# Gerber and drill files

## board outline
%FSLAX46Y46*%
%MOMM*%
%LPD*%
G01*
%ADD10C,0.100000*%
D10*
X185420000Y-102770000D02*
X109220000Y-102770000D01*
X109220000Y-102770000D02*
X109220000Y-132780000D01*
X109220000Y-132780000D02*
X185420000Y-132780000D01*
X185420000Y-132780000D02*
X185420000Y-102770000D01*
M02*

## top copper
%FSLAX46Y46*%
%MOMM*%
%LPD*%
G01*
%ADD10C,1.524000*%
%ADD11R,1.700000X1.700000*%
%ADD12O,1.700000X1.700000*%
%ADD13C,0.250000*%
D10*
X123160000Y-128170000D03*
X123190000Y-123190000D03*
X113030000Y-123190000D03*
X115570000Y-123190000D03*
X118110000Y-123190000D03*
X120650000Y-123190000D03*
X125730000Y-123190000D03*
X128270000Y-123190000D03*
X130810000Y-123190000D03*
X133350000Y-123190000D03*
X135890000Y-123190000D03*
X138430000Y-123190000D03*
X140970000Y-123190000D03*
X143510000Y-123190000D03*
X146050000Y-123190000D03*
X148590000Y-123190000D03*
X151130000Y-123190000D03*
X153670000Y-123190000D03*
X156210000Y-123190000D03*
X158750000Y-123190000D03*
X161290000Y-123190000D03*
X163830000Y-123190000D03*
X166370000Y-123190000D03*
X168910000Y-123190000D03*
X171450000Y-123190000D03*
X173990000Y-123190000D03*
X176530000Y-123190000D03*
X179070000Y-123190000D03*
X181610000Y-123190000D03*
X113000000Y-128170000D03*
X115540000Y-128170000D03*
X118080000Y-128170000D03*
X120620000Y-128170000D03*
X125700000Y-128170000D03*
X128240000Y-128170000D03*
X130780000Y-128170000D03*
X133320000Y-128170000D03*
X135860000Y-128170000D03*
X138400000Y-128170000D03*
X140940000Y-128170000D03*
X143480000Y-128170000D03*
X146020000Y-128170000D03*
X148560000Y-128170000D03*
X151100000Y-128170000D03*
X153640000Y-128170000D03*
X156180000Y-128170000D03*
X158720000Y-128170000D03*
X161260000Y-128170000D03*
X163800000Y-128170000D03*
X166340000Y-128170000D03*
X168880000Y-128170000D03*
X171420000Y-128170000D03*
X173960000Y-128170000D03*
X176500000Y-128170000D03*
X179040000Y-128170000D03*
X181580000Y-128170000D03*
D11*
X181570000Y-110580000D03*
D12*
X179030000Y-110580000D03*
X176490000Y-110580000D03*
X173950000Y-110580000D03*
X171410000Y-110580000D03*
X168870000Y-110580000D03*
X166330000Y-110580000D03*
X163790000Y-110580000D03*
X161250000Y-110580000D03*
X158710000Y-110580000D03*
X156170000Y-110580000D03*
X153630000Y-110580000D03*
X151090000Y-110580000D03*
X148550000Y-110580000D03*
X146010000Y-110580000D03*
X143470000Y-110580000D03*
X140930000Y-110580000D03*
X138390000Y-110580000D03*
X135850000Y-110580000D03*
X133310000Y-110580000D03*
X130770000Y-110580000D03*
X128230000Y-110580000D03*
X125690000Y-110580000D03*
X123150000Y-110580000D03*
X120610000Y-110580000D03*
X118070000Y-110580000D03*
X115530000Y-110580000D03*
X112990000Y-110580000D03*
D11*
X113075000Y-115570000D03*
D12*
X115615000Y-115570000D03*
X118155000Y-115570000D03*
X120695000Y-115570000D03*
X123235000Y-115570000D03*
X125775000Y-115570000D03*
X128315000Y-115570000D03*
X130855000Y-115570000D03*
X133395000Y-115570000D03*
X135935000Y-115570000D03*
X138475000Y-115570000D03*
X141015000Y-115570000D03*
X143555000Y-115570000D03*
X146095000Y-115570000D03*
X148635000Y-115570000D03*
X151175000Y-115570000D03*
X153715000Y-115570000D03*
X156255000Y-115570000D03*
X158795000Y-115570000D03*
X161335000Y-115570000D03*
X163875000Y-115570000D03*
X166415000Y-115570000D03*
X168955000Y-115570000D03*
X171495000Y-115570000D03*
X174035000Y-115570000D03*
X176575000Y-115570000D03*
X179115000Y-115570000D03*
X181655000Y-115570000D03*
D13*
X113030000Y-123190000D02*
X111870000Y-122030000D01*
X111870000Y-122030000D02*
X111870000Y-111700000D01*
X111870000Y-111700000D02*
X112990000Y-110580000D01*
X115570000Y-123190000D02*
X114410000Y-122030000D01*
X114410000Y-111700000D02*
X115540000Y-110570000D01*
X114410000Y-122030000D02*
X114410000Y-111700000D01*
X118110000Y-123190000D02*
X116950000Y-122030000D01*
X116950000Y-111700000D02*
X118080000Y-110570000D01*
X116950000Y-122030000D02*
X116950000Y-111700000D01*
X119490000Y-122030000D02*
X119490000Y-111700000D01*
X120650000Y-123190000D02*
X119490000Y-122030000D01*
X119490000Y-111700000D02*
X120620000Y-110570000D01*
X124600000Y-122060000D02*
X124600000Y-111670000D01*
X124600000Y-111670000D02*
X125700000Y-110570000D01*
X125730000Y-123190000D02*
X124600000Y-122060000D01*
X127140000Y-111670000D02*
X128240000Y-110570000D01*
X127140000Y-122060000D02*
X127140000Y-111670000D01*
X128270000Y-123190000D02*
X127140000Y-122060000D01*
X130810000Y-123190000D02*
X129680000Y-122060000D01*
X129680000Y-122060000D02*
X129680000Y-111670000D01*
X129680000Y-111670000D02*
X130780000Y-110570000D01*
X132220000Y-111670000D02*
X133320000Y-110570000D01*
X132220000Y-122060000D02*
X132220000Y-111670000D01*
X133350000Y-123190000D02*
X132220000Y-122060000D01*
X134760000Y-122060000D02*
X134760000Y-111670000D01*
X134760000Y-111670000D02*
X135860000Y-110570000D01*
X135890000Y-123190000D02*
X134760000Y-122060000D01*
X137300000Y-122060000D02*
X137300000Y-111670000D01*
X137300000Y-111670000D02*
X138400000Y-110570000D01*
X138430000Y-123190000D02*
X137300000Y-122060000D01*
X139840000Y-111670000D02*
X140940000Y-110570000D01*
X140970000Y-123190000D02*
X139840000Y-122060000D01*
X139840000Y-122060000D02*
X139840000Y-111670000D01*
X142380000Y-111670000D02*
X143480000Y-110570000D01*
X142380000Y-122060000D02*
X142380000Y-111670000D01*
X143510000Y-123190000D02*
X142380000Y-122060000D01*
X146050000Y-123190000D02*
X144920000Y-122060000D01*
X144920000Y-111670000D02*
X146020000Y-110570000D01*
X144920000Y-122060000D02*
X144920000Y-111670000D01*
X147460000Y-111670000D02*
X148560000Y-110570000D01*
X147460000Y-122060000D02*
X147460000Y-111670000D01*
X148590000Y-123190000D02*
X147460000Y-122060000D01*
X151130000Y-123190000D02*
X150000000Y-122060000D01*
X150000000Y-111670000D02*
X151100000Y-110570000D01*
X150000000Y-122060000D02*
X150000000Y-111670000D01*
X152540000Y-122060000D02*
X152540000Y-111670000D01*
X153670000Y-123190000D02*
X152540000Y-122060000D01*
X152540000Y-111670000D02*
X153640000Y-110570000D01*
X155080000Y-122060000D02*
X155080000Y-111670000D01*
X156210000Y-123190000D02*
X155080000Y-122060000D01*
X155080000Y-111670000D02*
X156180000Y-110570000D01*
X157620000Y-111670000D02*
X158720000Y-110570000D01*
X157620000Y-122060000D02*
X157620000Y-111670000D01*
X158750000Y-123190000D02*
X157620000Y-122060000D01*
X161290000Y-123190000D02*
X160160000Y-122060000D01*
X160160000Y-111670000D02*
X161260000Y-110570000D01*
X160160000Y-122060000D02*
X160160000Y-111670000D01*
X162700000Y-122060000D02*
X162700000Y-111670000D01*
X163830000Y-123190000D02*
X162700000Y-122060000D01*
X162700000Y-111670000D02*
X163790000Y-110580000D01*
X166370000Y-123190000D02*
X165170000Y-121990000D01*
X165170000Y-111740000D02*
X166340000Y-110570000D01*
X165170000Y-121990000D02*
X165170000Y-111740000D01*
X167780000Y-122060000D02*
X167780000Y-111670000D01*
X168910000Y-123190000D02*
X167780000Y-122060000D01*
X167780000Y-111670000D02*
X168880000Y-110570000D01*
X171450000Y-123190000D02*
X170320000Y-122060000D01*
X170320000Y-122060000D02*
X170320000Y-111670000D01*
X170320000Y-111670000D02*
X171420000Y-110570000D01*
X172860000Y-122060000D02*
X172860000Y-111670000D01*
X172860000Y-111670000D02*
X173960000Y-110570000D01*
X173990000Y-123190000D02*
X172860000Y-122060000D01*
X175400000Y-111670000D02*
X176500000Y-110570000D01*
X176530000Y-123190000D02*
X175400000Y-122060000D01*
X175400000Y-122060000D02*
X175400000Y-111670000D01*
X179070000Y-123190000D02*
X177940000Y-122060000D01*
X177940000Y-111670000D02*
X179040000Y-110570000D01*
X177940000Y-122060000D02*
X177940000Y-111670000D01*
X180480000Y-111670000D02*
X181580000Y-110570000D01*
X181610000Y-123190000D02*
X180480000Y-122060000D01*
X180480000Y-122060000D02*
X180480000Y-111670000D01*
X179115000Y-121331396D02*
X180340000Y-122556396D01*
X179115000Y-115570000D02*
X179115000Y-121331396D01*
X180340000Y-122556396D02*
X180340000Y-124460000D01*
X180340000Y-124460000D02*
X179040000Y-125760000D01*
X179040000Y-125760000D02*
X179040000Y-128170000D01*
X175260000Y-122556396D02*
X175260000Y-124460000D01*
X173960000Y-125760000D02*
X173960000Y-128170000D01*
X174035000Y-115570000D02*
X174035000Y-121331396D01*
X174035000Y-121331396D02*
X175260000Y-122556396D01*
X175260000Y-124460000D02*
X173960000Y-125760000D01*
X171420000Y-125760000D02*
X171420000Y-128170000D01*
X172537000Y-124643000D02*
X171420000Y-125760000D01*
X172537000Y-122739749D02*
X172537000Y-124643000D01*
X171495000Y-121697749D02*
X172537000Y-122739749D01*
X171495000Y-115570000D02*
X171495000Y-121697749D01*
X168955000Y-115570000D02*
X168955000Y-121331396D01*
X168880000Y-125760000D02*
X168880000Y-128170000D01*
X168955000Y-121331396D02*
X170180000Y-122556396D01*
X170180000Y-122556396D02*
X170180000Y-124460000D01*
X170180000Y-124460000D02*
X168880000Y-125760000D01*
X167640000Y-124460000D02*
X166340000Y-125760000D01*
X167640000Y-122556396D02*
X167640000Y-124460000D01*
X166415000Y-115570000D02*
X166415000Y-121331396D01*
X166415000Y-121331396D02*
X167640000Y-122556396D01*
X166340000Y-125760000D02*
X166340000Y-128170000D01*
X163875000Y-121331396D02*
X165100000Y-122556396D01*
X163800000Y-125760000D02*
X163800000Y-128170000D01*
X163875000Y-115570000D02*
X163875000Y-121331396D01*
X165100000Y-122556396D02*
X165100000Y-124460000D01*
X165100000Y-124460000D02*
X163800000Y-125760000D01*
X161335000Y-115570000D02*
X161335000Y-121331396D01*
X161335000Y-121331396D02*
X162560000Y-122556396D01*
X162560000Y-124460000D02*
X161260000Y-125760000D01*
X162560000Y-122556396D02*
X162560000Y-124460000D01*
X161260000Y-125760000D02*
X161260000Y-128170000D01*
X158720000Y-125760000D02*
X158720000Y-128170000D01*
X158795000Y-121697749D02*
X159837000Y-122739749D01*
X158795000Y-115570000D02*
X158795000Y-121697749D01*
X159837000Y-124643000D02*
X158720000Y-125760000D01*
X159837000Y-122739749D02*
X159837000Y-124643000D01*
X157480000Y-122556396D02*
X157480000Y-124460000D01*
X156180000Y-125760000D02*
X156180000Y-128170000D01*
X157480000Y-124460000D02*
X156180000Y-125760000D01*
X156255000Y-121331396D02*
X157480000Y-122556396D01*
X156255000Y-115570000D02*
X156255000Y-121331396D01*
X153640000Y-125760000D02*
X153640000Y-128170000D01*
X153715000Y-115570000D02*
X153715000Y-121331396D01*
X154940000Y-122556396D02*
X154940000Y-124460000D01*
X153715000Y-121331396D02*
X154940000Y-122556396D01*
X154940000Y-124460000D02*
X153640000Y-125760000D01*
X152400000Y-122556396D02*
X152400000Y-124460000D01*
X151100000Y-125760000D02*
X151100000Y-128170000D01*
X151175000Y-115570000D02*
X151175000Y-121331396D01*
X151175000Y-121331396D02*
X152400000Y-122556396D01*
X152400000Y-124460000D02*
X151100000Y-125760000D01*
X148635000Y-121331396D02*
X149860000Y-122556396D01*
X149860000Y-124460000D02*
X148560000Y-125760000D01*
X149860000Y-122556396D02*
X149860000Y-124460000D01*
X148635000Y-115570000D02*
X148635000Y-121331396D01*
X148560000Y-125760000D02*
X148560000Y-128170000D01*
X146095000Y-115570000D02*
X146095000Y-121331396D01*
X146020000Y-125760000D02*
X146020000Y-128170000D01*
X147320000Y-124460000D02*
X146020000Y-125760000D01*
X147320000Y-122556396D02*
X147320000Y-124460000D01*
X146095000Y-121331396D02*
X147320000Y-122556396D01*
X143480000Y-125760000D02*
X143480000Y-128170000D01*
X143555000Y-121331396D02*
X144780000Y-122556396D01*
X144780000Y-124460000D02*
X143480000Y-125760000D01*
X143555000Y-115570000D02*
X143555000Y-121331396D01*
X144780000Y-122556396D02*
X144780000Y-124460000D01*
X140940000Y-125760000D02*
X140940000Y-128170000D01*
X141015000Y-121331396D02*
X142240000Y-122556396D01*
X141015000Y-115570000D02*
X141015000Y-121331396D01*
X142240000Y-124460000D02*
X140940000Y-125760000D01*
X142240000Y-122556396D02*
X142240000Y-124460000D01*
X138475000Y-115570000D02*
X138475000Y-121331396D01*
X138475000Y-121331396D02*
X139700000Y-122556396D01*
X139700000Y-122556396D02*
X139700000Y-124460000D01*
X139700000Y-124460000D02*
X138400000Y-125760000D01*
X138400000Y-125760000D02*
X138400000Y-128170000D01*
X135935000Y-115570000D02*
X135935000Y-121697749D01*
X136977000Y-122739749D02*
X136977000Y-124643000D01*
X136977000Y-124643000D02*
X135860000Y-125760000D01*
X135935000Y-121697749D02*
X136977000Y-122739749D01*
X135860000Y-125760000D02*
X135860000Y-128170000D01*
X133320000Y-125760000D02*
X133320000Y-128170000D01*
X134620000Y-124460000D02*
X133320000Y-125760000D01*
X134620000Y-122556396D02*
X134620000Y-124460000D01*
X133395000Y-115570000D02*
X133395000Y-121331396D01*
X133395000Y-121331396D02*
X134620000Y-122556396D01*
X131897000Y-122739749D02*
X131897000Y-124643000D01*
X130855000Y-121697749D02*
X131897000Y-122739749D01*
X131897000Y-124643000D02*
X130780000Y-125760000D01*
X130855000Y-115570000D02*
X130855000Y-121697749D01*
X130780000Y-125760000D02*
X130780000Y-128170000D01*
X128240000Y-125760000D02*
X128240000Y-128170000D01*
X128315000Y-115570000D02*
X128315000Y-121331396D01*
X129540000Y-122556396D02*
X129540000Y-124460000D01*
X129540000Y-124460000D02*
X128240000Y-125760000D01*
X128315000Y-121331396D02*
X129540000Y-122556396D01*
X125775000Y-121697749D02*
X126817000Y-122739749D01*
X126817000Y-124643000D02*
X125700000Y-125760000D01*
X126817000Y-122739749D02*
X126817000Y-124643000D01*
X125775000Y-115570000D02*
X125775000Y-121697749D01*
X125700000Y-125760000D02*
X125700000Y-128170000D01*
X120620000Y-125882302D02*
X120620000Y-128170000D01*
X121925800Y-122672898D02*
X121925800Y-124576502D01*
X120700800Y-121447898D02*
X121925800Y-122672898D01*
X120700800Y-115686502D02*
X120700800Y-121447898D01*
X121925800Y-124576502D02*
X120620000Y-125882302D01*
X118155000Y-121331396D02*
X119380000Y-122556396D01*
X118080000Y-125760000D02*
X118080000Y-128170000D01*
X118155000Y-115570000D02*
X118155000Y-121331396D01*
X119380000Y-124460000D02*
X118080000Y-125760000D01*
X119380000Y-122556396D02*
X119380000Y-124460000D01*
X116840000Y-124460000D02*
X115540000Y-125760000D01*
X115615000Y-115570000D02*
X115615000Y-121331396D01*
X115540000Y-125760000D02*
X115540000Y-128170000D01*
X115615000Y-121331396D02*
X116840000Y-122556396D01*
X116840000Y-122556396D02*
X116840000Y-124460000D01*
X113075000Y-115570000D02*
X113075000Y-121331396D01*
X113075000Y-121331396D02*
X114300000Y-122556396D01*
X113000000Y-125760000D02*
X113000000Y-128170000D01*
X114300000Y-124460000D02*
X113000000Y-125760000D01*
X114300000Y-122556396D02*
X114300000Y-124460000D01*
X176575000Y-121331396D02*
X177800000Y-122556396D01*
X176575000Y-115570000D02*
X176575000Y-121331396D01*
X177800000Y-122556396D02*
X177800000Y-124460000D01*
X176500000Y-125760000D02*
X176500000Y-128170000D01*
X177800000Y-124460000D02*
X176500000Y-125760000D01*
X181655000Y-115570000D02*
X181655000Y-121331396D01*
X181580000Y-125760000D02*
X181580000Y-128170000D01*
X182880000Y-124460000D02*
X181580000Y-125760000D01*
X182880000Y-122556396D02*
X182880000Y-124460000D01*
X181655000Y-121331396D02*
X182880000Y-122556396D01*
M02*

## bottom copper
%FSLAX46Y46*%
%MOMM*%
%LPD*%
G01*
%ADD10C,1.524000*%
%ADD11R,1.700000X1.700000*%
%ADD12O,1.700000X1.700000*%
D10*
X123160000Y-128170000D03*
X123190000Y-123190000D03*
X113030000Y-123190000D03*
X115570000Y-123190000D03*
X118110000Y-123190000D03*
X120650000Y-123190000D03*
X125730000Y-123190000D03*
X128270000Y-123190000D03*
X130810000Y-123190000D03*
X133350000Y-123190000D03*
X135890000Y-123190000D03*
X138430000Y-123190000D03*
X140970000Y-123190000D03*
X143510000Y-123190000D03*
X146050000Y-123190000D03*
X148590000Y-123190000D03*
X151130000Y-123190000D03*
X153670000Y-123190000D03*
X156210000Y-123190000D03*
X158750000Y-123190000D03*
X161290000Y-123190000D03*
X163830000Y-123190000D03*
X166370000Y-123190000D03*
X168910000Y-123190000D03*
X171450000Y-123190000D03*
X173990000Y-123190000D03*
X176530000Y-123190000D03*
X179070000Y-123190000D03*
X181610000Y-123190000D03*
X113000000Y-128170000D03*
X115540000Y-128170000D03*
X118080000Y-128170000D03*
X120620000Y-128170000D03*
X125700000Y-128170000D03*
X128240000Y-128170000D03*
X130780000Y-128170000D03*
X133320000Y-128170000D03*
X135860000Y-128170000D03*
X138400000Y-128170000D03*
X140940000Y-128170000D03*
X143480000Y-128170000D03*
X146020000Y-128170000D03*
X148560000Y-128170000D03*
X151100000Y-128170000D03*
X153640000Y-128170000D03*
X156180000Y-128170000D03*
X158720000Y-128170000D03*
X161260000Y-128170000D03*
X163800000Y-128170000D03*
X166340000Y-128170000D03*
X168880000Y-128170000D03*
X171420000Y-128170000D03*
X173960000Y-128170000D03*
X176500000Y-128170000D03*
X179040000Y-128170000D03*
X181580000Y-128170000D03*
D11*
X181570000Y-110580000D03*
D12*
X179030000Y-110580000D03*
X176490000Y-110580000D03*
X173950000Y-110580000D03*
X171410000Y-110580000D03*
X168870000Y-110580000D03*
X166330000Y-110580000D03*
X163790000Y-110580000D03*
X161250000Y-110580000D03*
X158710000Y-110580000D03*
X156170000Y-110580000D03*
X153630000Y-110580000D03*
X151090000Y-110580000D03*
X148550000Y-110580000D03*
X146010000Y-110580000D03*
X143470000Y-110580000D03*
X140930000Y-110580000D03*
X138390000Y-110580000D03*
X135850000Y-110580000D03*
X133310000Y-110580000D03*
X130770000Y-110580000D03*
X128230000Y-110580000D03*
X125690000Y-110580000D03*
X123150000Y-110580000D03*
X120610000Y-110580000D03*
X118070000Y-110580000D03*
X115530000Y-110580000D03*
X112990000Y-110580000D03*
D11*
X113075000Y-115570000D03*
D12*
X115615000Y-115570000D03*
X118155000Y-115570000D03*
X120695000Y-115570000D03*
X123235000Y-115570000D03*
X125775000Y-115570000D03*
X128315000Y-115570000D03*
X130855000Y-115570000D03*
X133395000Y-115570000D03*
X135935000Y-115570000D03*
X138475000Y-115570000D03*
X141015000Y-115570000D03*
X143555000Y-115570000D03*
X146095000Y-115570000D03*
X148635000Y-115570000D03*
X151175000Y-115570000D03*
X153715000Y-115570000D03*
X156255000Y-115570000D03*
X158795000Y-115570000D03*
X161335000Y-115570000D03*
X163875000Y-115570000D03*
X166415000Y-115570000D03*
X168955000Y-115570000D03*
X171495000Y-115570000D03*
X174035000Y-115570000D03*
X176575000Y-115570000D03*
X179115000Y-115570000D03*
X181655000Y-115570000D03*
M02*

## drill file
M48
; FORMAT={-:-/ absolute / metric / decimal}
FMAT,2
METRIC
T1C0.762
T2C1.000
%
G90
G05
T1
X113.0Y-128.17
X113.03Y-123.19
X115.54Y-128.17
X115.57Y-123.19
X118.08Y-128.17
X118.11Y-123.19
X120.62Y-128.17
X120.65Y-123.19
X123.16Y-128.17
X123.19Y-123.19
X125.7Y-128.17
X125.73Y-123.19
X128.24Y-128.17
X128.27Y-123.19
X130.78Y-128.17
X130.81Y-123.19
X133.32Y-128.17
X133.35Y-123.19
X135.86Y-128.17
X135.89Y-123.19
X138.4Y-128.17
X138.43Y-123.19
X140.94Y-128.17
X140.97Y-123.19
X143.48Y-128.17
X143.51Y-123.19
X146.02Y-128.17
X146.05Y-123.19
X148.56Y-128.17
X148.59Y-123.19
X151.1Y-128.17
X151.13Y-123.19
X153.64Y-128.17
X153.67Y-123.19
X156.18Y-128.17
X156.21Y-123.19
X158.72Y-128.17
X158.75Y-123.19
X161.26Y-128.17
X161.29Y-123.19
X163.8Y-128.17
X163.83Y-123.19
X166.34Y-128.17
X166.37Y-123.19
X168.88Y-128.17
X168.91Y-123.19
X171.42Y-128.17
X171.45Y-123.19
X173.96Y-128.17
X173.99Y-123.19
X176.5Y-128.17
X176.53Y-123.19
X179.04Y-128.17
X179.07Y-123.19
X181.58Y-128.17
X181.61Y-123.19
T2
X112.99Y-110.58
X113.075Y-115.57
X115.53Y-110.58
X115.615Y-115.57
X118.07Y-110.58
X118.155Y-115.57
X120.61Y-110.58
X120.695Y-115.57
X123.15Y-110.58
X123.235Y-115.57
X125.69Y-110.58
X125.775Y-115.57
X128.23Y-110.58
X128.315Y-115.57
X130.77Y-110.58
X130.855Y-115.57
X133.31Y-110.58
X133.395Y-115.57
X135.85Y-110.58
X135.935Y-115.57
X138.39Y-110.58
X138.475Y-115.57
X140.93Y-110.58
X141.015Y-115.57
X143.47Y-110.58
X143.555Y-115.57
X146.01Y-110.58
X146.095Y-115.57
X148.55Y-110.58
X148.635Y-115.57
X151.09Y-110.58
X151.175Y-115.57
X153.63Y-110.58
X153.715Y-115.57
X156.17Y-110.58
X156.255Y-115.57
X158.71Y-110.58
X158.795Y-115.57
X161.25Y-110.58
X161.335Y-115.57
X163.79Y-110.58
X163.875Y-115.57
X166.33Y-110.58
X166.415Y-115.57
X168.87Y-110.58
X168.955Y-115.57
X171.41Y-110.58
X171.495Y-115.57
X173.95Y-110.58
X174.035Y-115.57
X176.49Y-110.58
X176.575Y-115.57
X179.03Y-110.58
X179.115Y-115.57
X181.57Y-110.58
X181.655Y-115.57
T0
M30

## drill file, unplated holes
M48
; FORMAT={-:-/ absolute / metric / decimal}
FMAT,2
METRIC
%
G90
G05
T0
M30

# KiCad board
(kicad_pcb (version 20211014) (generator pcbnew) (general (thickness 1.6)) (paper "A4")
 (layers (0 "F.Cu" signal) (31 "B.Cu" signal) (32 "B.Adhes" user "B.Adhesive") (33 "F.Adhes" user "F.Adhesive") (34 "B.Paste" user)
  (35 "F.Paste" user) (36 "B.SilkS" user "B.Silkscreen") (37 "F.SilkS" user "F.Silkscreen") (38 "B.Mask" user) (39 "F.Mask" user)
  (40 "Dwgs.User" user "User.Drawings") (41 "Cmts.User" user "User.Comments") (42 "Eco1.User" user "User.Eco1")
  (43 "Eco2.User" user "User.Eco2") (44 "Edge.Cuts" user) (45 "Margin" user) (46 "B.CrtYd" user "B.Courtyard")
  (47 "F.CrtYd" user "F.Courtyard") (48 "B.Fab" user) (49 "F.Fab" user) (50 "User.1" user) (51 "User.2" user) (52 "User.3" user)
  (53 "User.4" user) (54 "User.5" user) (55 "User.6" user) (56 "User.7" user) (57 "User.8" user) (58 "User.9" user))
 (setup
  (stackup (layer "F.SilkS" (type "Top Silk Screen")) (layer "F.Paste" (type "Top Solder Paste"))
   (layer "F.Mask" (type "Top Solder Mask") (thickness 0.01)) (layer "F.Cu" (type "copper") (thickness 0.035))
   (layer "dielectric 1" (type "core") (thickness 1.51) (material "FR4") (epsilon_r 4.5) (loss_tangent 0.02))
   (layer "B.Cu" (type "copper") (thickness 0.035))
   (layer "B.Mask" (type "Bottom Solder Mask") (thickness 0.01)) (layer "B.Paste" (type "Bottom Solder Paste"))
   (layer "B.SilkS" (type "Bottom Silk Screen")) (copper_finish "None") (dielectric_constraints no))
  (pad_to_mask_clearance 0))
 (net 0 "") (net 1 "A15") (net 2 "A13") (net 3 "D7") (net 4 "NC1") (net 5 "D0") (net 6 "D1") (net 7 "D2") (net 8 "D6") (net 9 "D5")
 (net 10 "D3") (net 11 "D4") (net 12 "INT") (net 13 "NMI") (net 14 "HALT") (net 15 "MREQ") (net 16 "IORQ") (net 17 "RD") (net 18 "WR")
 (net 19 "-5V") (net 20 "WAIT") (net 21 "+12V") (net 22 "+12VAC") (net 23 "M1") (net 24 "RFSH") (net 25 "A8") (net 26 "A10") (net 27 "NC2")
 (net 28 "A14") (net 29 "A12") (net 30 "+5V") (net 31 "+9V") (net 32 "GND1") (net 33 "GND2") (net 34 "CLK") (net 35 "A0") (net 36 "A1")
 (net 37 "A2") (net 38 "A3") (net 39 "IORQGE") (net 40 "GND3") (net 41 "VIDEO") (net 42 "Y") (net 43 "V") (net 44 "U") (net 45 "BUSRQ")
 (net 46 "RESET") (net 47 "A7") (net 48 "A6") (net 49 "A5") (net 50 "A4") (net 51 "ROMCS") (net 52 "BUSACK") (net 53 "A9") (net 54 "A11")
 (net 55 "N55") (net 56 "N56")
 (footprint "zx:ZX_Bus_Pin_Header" (layer "F.Cu") (at 147.32 124.46)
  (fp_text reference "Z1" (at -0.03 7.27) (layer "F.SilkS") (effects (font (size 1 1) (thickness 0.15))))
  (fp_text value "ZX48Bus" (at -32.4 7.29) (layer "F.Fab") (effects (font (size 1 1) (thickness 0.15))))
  (pad "" thru_hole circle (at -24.16 3.71) (size 1.524 1.524) (drill 0.762) (layers *.Cu *.Mask))
  (pad "" thru_hole circle (at -24.13 -1.27) (size 1.524 1.524) (drill 0.762) (layers *.Cu *.Mask))
  (pad "A1" thru_hole circle (at -34.29 -1.27) (size 1.524 1.524) (drill 0.762) (layers *.Cu *.Mask) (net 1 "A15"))
  (pad "A2" thru_hole circle (at -31.75 -1.27) (size 1.524 1.524) (drill 0.762) (layers *.Cu *.Mask) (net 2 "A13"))
  (pad "A3" thru_hole circle (at -29.21 -1.27) (size 1.524 1.524) (drill 0.762) (layers *.Cu *.Mask) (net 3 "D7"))
  (pad "A4" thru_hole circle (at -26.67 -1.27) (size 1.524 1.524) (drill 0.762) (layers *.Cu *.Mask) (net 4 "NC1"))
  (pad "A6" thru_hole circle (at -21.59 -1.27) (size 1.524 1.524) (drill 0.762) (layers *.Cu *.Mask) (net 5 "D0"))
  (pad "A7" thru_hole circle (at -19.05 -1.27) (size 1.524 1.524) (drill 0.762) (layers *.Cu *.Mask) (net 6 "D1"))
  (pad "A8" thru_hole circle (at -16.51 -1.27) (size 1.524 1.524) (drill 0.762) (layers *.Cu *.Mask) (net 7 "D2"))
  (pad "A9" thru_hole circle (at -13.97 -1.27) (size 1.524 1.524) (drill 0.762) (layers *.Cu *.Mask) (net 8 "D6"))
  (pad "A10" thru_hole circle (at -11.43 -1.27) (size 1.524 1.524) (drill 0.762) (layers *.Cu *.Mask) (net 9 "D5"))
  (pad "A11" thru_hole circle (at -8.89 -1.27) (size 1.524 1.524) (drill 0.762) (layers *.Cu *.Mask) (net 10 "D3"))
  (pad "A12" thru_hole circle (at -6.35 -1.27) (size 1.524 1.524) (drill 0.762) (layers *.Cu *.Mask) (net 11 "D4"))
  (pad "A13" thru_hole circle (at -3.81 -1.27) (size 1.524 1.524) (drill 0.762) (layers *.Cu *.Mask) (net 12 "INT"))
  (pad "A14" thru_hole circle (at -1.27 -1.27) (size 1.524 1.524) (drill 0.762) (layers *.Cu *.Mask) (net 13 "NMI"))
  (pad "A15" thru_hole circle (at 1.27 -1.27) (size 1.524 1.524) (drill 0.762) (layers *.Cu *.Mask) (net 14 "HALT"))
  (pad "A16" thru_hole circle (at 3.81 -1.27) (size 1.524 1.524) (drill 0.762) (layers *.Cu *.Mask) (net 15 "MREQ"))
  (pad "A17" thru_hole circle (at 6.35 -1.27) (size 1.524 1.524) (drill 0.762) (layers *.Cu *.Mask) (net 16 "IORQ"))
  (pad "A18" thru_hole circle (at 8.89 -1.27) (size 1.524 1.524) (drill 0.762) (layers *.Cu *.Mask) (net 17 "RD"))
  (pad "A19" thru_hole circle (at 11.43 -1.27) (size 1.524 1.524) (drill 0.762) (layers *.Cu *.Mask) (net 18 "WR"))
  (pad "A20" thru_hole circle (at 13.97 -1.27) (size 1.524 1.524) (drill 0.762) (layers *.Cu *.Mask) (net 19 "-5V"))
  (pad "A21" thru_hole circle (at 16.51 -1.27) (size 1.524 1.524) (drill 0.762) (layers *.Cu *.Mask) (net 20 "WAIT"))
  (pad "A22" thru_hole circle (at 19.05 -1.27) (size 1.524 1.524) (drill 0.762) (layers *.Cu *.Mask) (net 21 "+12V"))
  (pad "A23" thru_hole circle (at 21.59 -1.27) (size 1.524 1.524) (drill 0.762) (layers *.Cu *.Mask) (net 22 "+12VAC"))
  (pad "A24" thru_hole circle (at 24.13 -1.27) (size 1.524 1.524) (drill 0.762) (layers *.Cu *.Mask) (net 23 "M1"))
  (pad "A25" thru_hole circle (at 26.67 -1.27) (size 1.524 1.524) (drill 0.762) (layers *.Cu *.Mask) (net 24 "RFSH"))
  (pad "A26" thru_hole circle (at 29.21 -1.27) (size 1.524 1.524) (drill 0.762) (layers *.Cu *.Mask) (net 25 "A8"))
  (pad "A27" thru_hole circle (at 31.75 -1.27) (size 1.524 1.524) (drill 0.762) (layers *.Cu *.Mask) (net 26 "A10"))
  (pad "A28" thru_hole circle (at 34.29 -1.27) (size 1.524 1.524) (drill 0.762) (layers *.Cu *.Mask) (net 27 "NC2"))
  (pad "B1" thru_hole circle (at -34.32 3.71) (size 1.524 1.524) (drill 0.762) (layers *.Cu *.Mask) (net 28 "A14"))
  (pad "B2" thru_hole circle (at -31.78 3.71) (size 1.524 1.524) (drill 0.762) (layers *.Cu *.Mask) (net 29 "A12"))
  (pad "B3" thru_hole circle (at -29.24 3.71) (size 1.524 1.524) (drill 0.762) (layers *.Cu *.Mask) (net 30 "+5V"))
  (pad "B4" thru_hole circle (at -26.7 3.71) (size 1.524 1.524) (drill 0.762) (layers *.Cu *.Mask) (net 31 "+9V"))
  (pad "B6" thru_hole circle (at -21.62 3.71) (size 1.524 1.524) (drill 0.762) (layers *.Cu *.Mask) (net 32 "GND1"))
  (pad "B7" thru_hole circle (at -19.08 3.71) (size 1.524 1.524) (drill 0.762) (layers *.Cu *.Mask) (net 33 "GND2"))
  (pad "B8" thru_hole circle (at -16.54 3.71) (size 1.524 1.524) (drill 0.762) (layers *.Cu *.Mask) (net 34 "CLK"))
  (pad "B9" thru_hole circle (at -14 3.71) (size 1.524 1.524) (drill 0.762) (layers *.Cu *.Mask) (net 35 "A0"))
  (pad "B10" thru_hole circle (at -11.46 3.71) (size 1.524 1.524) (drill 0.762) (layers *.Cu *.Mask) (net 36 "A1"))
  (pad "B11" thru_hole circle (at -8.92 3.71) (size 1.524 1.524) (drill 0.762) (layers *.Cu *.Mask) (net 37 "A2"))
  (pad "B12" thru_hole circle (at -6.38 3.71) (size 1.524 1.524) (drill 0.762) (layers *.Cu *.Mask) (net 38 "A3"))
  (pad "B13" thru_hole circle (at -3.84 3.71) (size 1.524 1.524) (drill 0.762) (layers *.Cu *.Mask) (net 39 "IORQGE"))
  (pad "B14" thru_hole circle (at -1.3 3.71) (size 1.524 1.524) (drill 0.762) (layers *.Cu *.Mask) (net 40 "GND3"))
  (pad "B15" thru_hole circle (at 1.24 3.71) (size 1.524 1.524) (drill 0.762) (layers *.Cu *.Mask) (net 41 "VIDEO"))
  (pad "B16" thru_hole circle (at 3.78 3.71) (size 1.524 1.524) (drill 0.762) (layers *.Cu *.Mask) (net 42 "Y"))
  (pad "B17" thru_hole circle (at 6.32 3.71) (size 1.524 1.524) (drill 0.762) (layers *.Cu *.Mask) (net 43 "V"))
  (pad "B18" thru_hole circle (at 8.86 3.71) (size 1.524 1.524) (drill 0.762) (layers *.Cu *.Mask) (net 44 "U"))
  (pad "B19" thru_hole circle (at 11.4 3.71) (size 1.524 1.524) (drill 0.762) (layers *.Cu *.Mask) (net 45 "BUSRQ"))
  (pad "B20" thru_hole circle (at 13.94 3.71) (size 1.524 1.524) (drill 0.762) (layers *.Cu *.Mask) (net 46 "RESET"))
  (pad "B21" thru_hole circle (at 16.48 3.71) (size 1.524 1.524) (drill 0.762) (layers *.Cu *.Mask) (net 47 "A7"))
  (pad "B22" thru_hole circle (at 19.02 3.71) (size 1.524 1.524) (drill 0.762) (layers *.Cu *.Mask) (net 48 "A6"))
  (pad "B23" thru_hole circle (at 21.56 3.71) (size 1.524 1.524) (drill 0.762) (layers *.Cu *.Mask) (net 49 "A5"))
  (pad "B24" thru_hole circle (at 24.1 3.71) (size 1.524 1.524) (drill 0.762) (layers *.Cu *.Mask) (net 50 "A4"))
  (pad "B25" thru_hole circle (at 26.64 3.71) (size 1.524 1.524) (drill 0.762) (layers *.Cu *.Mask) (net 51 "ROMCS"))
  (pad "B26" thru_hole circle (at 29.18 3.71) (size 1.524 1.524) (drill 0.762) (layers *.Cu *.Mask) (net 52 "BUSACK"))
  (pad "B27" thru_hole circle (at 31.72 3.71) (size 1.524 1.524) (drill 0.762) (layers *.Cu *.Mask) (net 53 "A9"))
  (pad "B28" thru_hole circle (at 34.26 3.71) (size 1.524 1.524) (drill 0.762) (layers *.Cu *.Mask) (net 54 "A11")))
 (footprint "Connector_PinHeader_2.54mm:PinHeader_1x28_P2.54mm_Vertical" (layer "B.Cu") (at 181.57 110.58 90)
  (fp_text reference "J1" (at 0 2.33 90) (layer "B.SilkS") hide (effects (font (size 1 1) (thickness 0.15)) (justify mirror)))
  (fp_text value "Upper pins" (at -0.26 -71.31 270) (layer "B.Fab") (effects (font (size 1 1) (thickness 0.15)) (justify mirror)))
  (pad "1" thru_hole rect (at 0 0 90) (size 1.7 1.7) (drill 1) (layers *.Cu *.Mask) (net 27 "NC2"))
  (pad "2" thru_hole oval (at 0 -2.54 90) (size 1.7 1.7) (drill 1) (layers *.Cu *.Mask) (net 26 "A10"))
  (pad "3" thru_hole oval (at 0 -5.08 90) (size 1.7 1.7) (drill 1) (layers *.Cu *.Mask) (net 25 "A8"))
  (pad "4" thru_hole oval (at 0 -7.62 90) (size 1.7 1.7) (drill 1) (layers *.Cu *.Mask) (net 24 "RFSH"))
  (pad "5" thru_hole oval (at 0 -10.16 90) (size 1.7 1.7) (drill 1) (layers *.Cu *.Mask) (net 23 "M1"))
  (pad "6" thru_hole oval (at 0 -12.7 90) (size 1.7 1.7) (drill 1) (layers *.Cu *.Mask) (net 22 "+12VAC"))
  (pad "7" thru_hole oval (at 0 -15.24 90) (size 1.7 1.7) (drill 1) (layers *.Cu *.Mask) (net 21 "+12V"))
  (pad "8" thru_hole oval (at 0 -17.78 90) (size 1.7 1.7) (drill 1) (layers *.Cu *.Mask) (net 20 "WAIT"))
  (pad "9" thru_hole oval (at 0 -20.32 90) (size 1.7 1.7) (drill 1) (layers *.Cu *.Mask) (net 19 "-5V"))
  (pad "10" thru_hole oval (at 0 -22.86 90) (size 1.7 1.7) (drill 1) (layers *.Cu *.Mask) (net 18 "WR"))
  (pad "11" thru_hole oval (at 0 -25.4 90) (size 1.7 1.7) (drill 1) (layers *.Cu *.Mask) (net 17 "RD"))
  (pad "12" thru_hole oval (at 0 -27.94 90) (size 1.7 1.7) (drill 1) (layers *.Cu *.Mask) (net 16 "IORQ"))
  (pad "13" thru_hole oval (at 0 -30.48 90) (size 1.7 1.7) (drill 1) (layers *.Cu *.Mask) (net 15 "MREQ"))
  (pad "14" thru_hole oval (at 0 -33.02 90) (size 1.7 1.7) (drill 1) (layers *.Cu *.Mask) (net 14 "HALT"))
  (pad "15" thru_hole oval (at 0 -35.56 90) (size 1.7 1.7) (drill 1) (layers *.Cu *.Mask) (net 13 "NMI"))
  (pad "16" thru_hole oval (at 0 -38.1 90) (size 1.7 1.7) (drill 1) (layers *.Cu *.Mask) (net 12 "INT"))
  (pad "17" thru_hole oval (at 0 -40.64 90) (size 1.7 1.7) (drill 1) (layers *.Cu *.Mask) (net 11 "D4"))
  (pad "18" thru_hole oval (at 0 -43.18 90) (size 1.7 1.7) (drill 1) (layers *.Cu *.Mask) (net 10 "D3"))
  (pad "19" thru_hole oval (at 0 -45.72 90) (size 1.7 1.7) (drill 1) (layers *.Cu *.Mask) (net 9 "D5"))
  (pad "20" thru_hole oval (at 0 -48.26 90) (size 1.7 1.7) (drill 1) (layers *.Cu *.Mask) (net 8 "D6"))
  (pad "21" thru_hole oval (at 0 -50.8 90) (size 1.7 1.7) (drill 1) (layers *.Cu *.Mask) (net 7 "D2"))
  (pad "22" thru_hole oval (at 0 -53.34 90) (size 1.7 1.7) (drill 1) (layers *.Cu *.Mask) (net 6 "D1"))
  (pad "23" thru_hole oval (at 0 -55.88 90) (size 1.7 1.7) (drill 1) (layers *.Cu *.Mask) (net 5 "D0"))
  (pad "24" thru_hole oval (at 0 -58.42 90) (size 1.7 1.7) (drill 1) (layers *.Cu *.Mask) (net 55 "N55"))
  (pad "25" thru_hole oval (at 0 -60.96 90) (size 1.7 1.7) (drill 1) (layers *.Cu *.Mask) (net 4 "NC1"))
  (pad "26" thru_hole oval (at 0 -63.5 90) (size 1.7 1.7) (drill 1) (layers *.Cu *.Mask) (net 3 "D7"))
  (pad "27" thru_hole oval (at 0 -66.04 90) (size 1.7 1.7) (drill 1) (layers *.Cu *.Mask) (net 2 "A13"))
  (pad "28" thru_hole oval (at 0 -68.58 90) (size 1.7 1.7) (drill 1) (layers *.Cu *.Mask) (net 1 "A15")))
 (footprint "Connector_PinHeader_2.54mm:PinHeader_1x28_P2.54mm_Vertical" (layer "B.Cu") (at 113.075 115.57 -90)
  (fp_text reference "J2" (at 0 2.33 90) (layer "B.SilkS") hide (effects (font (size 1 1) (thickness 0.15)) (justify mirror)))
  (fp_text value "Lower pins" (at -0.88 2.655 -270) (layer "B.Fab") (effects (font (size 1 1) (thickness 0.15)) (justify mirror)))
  (pad "1" thru_hole rect (at 0 0 270) (size 1.7 1.7) (drill 1) (layers *.Cu *.Mask) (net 28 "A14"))
  (pad "2" thru_hole oval (at 0 -2.54 270) (size 1.7 1.7) (drill 1) (layers *.Cu *.Mask) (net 29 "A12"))
  (pad "3" thru_hole oval (at 0 -5.08 270) (size 1.7 1.7) (drill 1) (layers *.Cu *.Mask) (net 30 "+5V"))
  (pad "4" thru_hole oval (at 0 -7.62 270) (size 1.7 1.7) (drill 1) (layers *.Cu *.Mask) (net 31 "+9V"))
  (pad "5" thru_hole oval (at 0 -10.16 270) (size 1.7 1.7) (drill 1) (layers *.Cu *.Mask) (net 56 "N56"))
  (pad "6" thru_hole oval (at 0 -12.7 270) (size 1.7 1.7) (drill 1) (layers *.Cu *.Mask) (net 32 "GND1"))
  (pad "7" thru_hole oval (at 0 -15.24 270) (size 1.7 1.7) (drill 1) (layers *.Cu *.Mask) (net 33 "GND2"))
  (pad "8" thru_hole oval (at 0 -17.78 270) (size 1.7 1.7) (drill 1) (layers *.Cu *.Mask) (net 34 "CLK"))
  (pad "9" thru_hole oval (at 0 -20.32 270) (size 1.7 1.7) (drill 1) (layers *.Cu *.Mask) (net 35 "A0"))
  (pad "10" thru_hole oval (at 0 -22.86 270) (size 1.7 1.7) (drill 1) (layers *.Cu *.Mask) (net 36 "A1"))
  (pad "11" thru_hole oval (at 0 -25.4 270) (size 1.7 1.7) (drill 1) (layers *.Cu *.Mask) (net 37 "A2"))
  (pad "12" thru_hole oval (at 0 -27.94 270) (size 1.7 1.7) (drill 1) (layers *.Cu *.Mask) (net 38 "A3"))
  (pad "13" thru_hole oval (at 0 -30.48 270) (size 1.7 1.7) (drill 1) (layers *.Cu *.Mask) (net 39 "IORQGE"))
  (pad "14" thru_hole oval (at 0 -33.02 270) (size 1.7 1.7) (drill 1) (layers *.Cu *.Mask) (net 40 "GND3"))
  (pad "15" thru_hole oval (at 0 -35.56 270) (size 1.7 1.7) (drill 1) (layers *.Cu *.Mask) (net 41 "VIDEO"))
  (pad "16" thru_hole oval (at 0 -38.1 270) (size 1.7 1.7) (drill 1) (layers *.Cu *.Mask) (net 42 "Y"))
  (pad "17" thru_hole oval (at 0 -40.64 270) (size 1.7 1.7) (drill 1) (layers *.Cu *.Mask) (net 43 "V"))
  (pad "18" thru_hole oval (at 0 -43.18 270) (size 1.7 1.7) (drill 1) (layers *.Cu *.Mask) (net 44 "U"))
  (pad "19" thru_hole oval (at 0 -45.72 270) (size 1.7 1.7) (drill 1) (layers *.Cu *.Mask) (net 45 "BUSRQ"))
  (pad "20" thru_hole oval (at 0 -48.26 270) (size 1.7 1.7) (drill 1) (layers *.Cu *.Mask) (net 46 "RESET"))
  (pad "21" thru_hole oval (at 0 -50.8 270) (size 1.7 1.7) (drill 1) (layers *.Cu *.Mask) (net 47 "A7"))
  (pad "22" thru_hole oval (at 0 -53.34 270) (size 1.7 1.7) (drill 1) (layers *.Cu *.Mask) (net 48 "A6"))
  (pad "23" thru_hole oval (at 0 -55.88 270) (size 1.7 1.7) (drill 1) (layers *.Cu *.Mask) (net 49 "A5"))
  (pad "24" thru_hole oval (at 0 -58.42 270) (size 1.7 1.7) (drill 1) (layers *.Cu *.Mask) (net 50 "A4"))
  (pad "25" thru_hole oval (at 0 -60.96 270) (size 1.7 1.7) (drill 1) (layers *.Cu *.Mask) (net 51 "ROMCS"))
  (pad "26" thru_hole oval (at 0 -63.5 270) (size 1.7 1.7) (drill 1) (layers *.Cu *.Mask) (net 52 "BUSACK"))
  (pad "27" thru_hole oval (at 0 -66.04 270) (size 1.7 1.7) (drill 1) (layers *.Cu *.Mask) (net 53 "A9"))
  (pad "28" thru_hole oval (at 0 -68.58 270) (size 1.7 1.7) (drill 1) (layers *.Cu *.Mask) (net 54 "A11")))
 (gr_rect (start 185.42 102.77) (end 109.22 132.78) (layer "Edge.Cuts") (width 0.1) (fill none))
 (segment (start 113.03 123.19) (end 111.87 122.03) (width 0.25) (layer "F.Cu") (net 1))
 (segment (start 111.87 122.03) (end 111.87 111.7) (width 0.25) (layer "F.Cu") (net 1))
 (segment (start 111.87 111.7) (end 112.99 110.58) (width 0.25) (layer "F.Cu") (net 1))
 (segment (start 115.57 123.19) (end 114.41 122.03) (width 0.25) (layer "F.Cu") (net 2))
 (segment (start 114.41 111.7) (end 115.54 110.57) (width 0.25) (layer "F.Cu") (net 2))
 (segment (start 114.41 122.03) (end 114.41 111.7) (width 0.25) (layer "F.Cu") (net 2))
 (segment (start 118.11 123.19) (end 116.95 122.03) (width 0.25) (layer "F.Cu") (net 3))
 (segment (start 116.95 111.7) (end 118.08 110.57) (width 0.25) (layer "F.Cu") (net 3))
 (segment (start 116.95 122.03) (end 116.95 111.7) (width 0.25) (layer "F.Cu") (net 3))
 (segment (start 119.49 122.03) (end 119.49 111.7) (width 0.25) (layer "F.Cu") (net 4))
 (segment (start 120.65 123.19) (end 119.49 122.03) (width 0.25) (layer "F.Cu") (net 4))
 (segment (start 119.49 111.7) (end 120.62 110.57) (width 0.25) (layer "F.Cu") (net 4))
 (segment (start 124.6 122.06) (end 124.6 111.67) (width 0.25) (layer "F.Cu") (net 5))
 (segment (start 124.6 111.67) (end 125.7 110.57) (width 0.25) (layer "F.Cu") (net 5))
 (segment (start 125.73 123.19) (end 124.6 122.06) (width 0.25) (layer "F.Cu") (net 5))
 (segment (start 127.14 111.67) (end 128.24 110.57) (width 0.25) (layer "F.Cu") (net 6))
 (segment (start 127.14 122.06) (end 127.14 111.67) (width 0.25) (layer "F.Cu") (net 6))
 (segment (start 128.27 123.19) (end 127.14 122.06) (width 0.25) (layer "F.Cu") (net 6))
 (segment (start 130.81 123.19) (end 129.68 122.06) (width 0.25) (layer "F.Cu") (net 7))
 (segment (start 129.68 122.06) (end 129.68 111.67) (width 0.25) (layer "F.Cu") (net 7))
 (segment (start 129.68 111.67) (end 130.78 110.57) (width 0.25) (layer "F.Cu") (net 7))
 (segment (start 132.22 111.67) (end 133.32 110.57) (width 0.25) (layer "F.Cu") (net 8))
 (segment (start 132.22 122.06) (end 132.22 111.67) (width 0.25) (layer "F.Cu") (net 8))
 (segment (start 133.35 123.19) (end 132.22 122.06) (width 0.25) (layer "F.Cu") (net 8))
 (segment (start 134.76 122.06) (end 134.76 111.67) (width 0.25) (layer "F.Cu") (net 9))
 (segment (start 134.76 111.67) (end 135.86 110.57) (width 0.25) (layer "F.Cu") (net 9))
 (segment (start 135.89 123.19) (end 134.76 122.06) (width 0.25) (layer "F.Cu") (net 9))
 (segment (start 137.3 122.06) (end 137.3 111.67) (width 0.25) (layer "F.Cu") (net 10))
 (segment (start 137.3 111.67) (end 138.4 110.57) (width 0.25) (layer "F.Cu") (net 10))
 (segment (start 138.43 123.19) (end 137.3 122.06) (width 0.25) (layer "F.Cu") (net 10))
 (segment (start 139.84 111.67) (end 140.94 110.57) (width 0.25) (layer "F.Cu") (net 11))
 (segment (start 140.97 123.19) (end 139.84 122.06) (width 0.25) (layer "F.Cu") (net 11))
 (segment (start 139.84 122.06) (end 139.84 111.67) (width 0.25) (layer "F.Cu") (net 11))
 (segment (start 142.38 111.67) (end 143.48 110.57) (width 0.25) (layer "F.Cu") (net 12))
 (segment (start 142.38 122.06) (end 142.38 111.67) (width 0.25) (layer "F.Cu") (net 12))
 (segment (start 143.51 123.19) (end 142.38 122.06) (width 0.25) (layer "F.Cu") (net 12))
 (segment (start 146.05 123.19) (end 144.92 122.06) (width 0.25) (layer "F.Cu") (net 13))
 (segment (start 144.92 111.67) (end 146.02 110.57) (width 0.25) (layer "F.Cu") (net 13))
 (segment (start 144.92 122.06) (end 144.92 111.67) (width 0.25) (layer "F.Cu") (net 13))
 (segment (start 147.46 111.67) (end 148.56 110.57) (width 0.25) (layer "F.Cu") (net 14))
 (segment (start 147.46 122.06) (end 147.46 111.67) (width 0.25) (layer "F.Cu") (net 14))
 (segment (start 148.59 123.19) (end 147.46 122.06) (width 0.25) (layer "F.Cu") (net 14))
 (segment (start 151.13 123.19) (end 150 122.06) (width 0.25) (layer "F.Cu") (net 15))
 (segment (start 150 111.67) (end 151.1 110.57) (width 0.25) (layer "F.Cu") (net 15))
 (segment (start 150 122.06) (end 150 111.67) (width 0.25) (layer "F.Cu") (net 15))
 (segment (start 152.54 122.06) (end 152.54 111.67) (width 0.25) (layer "F.Cu") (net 16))
 (segment (start 153.67 123.19) (end 152.54 122.06) (width 0.25) (layer "F.Cu") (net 16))
 (segment (start 152.54 111.67) (end 153.64 110.57) (width 0.25) (layer "F.Cu") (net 16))
 (segment (start 155.08 122.06) (end 155.08 111.67) (width 0.25) (layer "F.Cu") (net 17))
 (segment (start 156.21 123.19) (end 155.08 122.06) (width 0.25) (layer "F.Cu") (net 17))
 (segment (start 155.08 111.67) (end 156.18 110.57) (width 0.25) (layer "F.Cu") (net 17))
 (segment (start 157.62 111.67) (end 158.72 110.57) (width 0.25) (layer "F.Cu") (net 18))
 (segment (start 157.62 122.06) (end 157.62 111.67) (width 0.25) (layer "F.Cu") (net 18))
 (segment (start 158.75 123.19) (end 157.62 122.06) (width 0.25) (layer "F.Cu") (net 18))
 (segment (start 161.29 123.19) (end 160.16 122.06) (width 0.25) (layer "F.Cu") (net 19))
 (segment (start 160.16 111.67) (end 161.26 110.57) (width 0.25) (layer "F.Cu") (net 19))
 (segment (start 160.16 122.06) (end 160.16 111.67) (width 0.25) (layer "F.Cu") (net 19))
 (segment (start 162.7 122.06) (end 162.7 111.67) (width 0.25) (layer "F.Cu") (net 20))
 (segment (start 163.83 123.19) (end 162.7 122.06) (width 0.25) (layer "F.Cu") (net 20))
 (segment (start 162.7 111.67) (end 163.79 110.58) (width 0.25) (layer "F.Cu") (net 20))
 (segment (start 166.37 123.19) (end 165.17 121.99) (width 0.25) (layer "F.Cu") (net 21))
 (segment (start 165.17 111.74) (end 166.34 110.57) (width 0.25) (layer "F.Cu") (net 21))
 (segment (start 165.17 121.99) (end 165.17 111.74) (width 0.25) (layer "F.Cu") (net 21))
 (segment (start 167.78 122.06) (end 167.78 111.67) (width 0.25) (layer "F.Cu") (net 22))
 (segment (start 168.91 123.19) (end 167.78 122.06) (width 0.25) (layer "F.Cu") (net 22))
 (segment (start 167.78 111.67) (end 168.88 110.57) (width 0.25) (layer "F.Cu") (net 22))
 (segment (start 171.45 123.19) (end 170.32 122.06) (width 0.25) (layer "F.Cu") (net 23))
 (segment (start 170.32 122.06) (end 170.32 111.67) (width 0.25) (layer "F.Cu") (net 23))
 (segment (start 170.32 111.67) (end 171.42 110.57) (width 0.25) (layer "F.Cu") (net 23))
 (segment (start 172.86 122.06) (end 172.86 111.67) (width 0.25) (layer "F.Cu") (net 24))
 (segment (start 172.86 111.67) (end 173.96 110.57) (width 0.25) (layer "F.Cu") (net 24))
 (segment (start 173.99 123.19) (end 172.86 122.06) (width 0.25) (layer "F.Cu") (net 24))
 (segment (start 175.4 111.67) (end 176.5 110.57) (width 0.25) (layer "F.Cu") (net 25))
 (segment (start 176.53 123.19) (end 175.4 122.06) (width 0.25) (layer "F.Cu") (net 25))
 (segment (start 175.4 122.06) (end 175.4 111.67) (width 0.25) (layer "F.Cu") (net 25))
 (segment (start 179.07 123.19) (end 177.94 122.06) (width 0.25) (layer "F.Cu") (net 26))
 (segment (start 177.94 111.67) (end 179.04 110.57) (width 0.25) (layer "F.Cu") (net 26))
 (segment (start 177.94 122.06) (end 177.94 111.67) (width 0.25) (layer "F.Cu") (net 26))
 (segment (start 180.48 111.67) (end 181.58 110.57) (width 0.25) (layer "F.Cu") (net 27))
 (segment (start 181.61 123.19) (end 180.48 122.06) (width 0.25) (layer "F.Cu") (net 27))
 (segment (start 180.48 122.06) (end 180.48 111.67) (width 0.25) (layer "F.Cu") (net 27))
 (segment (start 179.115 121.331396) (end 180.34 122.556396) (width 0.25) (layer "F.Cu") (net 53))
 (segment (start 179.115 115.57) (end 179.115 121.331396) (width 0.25) (layer "F.Cu") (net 53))
 (segment (start 180.34 122.556396) (end 180.34 124.46) (width 0.25) (layer "F.Cu") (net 53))
 (segment (start 180.34 124.46) (end 179.04 125.76) (width 0.25) (layer "F.Cu") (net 53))
 (segment (start 179.04 125.76) (end 179.04 128.17) (width 0.25) (layer "F.Cu") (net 53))
 (segment (start 175.26 122.556396) (end 175.26 124.46) (width 0.25) (layer "F.Cu") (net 51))
 (segment (start 173.96 125.76) (end 173.96 128.17) (width 0.25) (layer "F.Cu") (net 51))
 (segment (start 174.035 115.57) (end 174.035 121.331396) (width 0.25) (layer "F.Cu") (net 51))
 (segment (start 174.035 121.331396) (end 175.26 122.556396) (width 0.25) (layer "F.Cu") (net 51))
 (segment (start 175.26 124.46) (end 173.96 125.76) (width 0.25) (layer "F.Cu") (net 51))
 (segment (start 171.42 125.76) (end 171.42 128.17) (width 0.25) (layer "F.Cu") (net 50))
 (segment (start 172.537 124.643) (end 171.42 125.76) (width 0.25) (layer "F.Cu") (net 50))
 (segment (start 172.537 122.739749) (end 172.537 124.643) (width 0.25) (layer "F.Cu") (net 50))
 (segment (start 171.495 121.697749) (end 172.537 122.739749) (width 0.25) (layer "F.Cu") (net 50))
 (segment (start 171.495 115.57) (end 171.495 121.697749) (width 0.25) (layer "F.Cu") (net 50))
 (segment (start 168.955 115.57) (end 168.955 121.331396) (width 0.25) (layer "F.Cu") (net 49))
 (segment (start 168.88 125.76) (end 168.88 128.17) (width 0.25) (layer "F.Cu") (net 49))
 (segment (start 168.955 121.331396) (end 170.18 122.556396) (width 0.25) (layer "F.Cu") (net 49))
 (segment (start 170.18 122.556396) (end 170.18 124.46) (width 0.25) (layer "F.Cu") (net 49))
 (segment (start 170.18 124.46) (end 168.88 125.76) (width 0.25) (layer "F.Cu") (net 49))
 (segment (start 167.64 124.46) (end 166.34 125.76) (width 0.25) (layer "F.Cu") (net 48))
 (segment (start 167.64 122.556396) (end 167.64 124.46) (width 0.25) (layer "F.Cu") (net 48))
 (segment (start 166.415 115.57) (end 166.415 121.331396) (width 0.25) (layer "F.Cu") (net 48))
 (segment (start 166.415 121.331396) (end 167.64 122.556396) (width 0.25) (layer "F.Cu") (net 48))
 (segment (start 166.34 125.76) (end 166.34 128.17) (width 0.25) (layer "F.Cu") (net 48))
 (segment (start 163.875 121.331396) (end 165.1 122.556396) (width 0.25) (layer "F.Cu") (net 47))
 (segment (start 163.8 125.76) (end 163.8 128.17) (width 0.25) (layer "F.Cu") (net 47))
 (segment (start 163.875 115.57) (end 163.875 121.331396) (width 0.25) (layer "F.Cu") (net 47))
 (segment (start 165.1 122.556396) (end 165.1 124.46) (width 0.25) (layer "F.Cu") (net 47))
 (segment (start 165.1 124.46) (end 163.8 125.76) (width 0.25) (layer "F.Cu") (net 47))
 (segment (start 161.335 115.57) (end 161.335 121.331396) (width 0.25) (layer "F.Cu") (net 46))
 (segment (start 161.335 121.331396) (end 162.56 122.556396) (width 0.25) (layer "F.Cu") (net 46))
 (segment (start 162.56 124.46) (end 161.26 125.76) (width 0.25) (layer "F.Cu") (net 46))
 (segment (start 162.56 122.556396) (end 162.56 124.46) (width 0.25) (layer "F.Cu") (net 46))
 (segment (start 161.26 125.76) (end 161.26 128.17) (width 0.25) (layer "F.Cu") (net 46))
 (segment (start 158.72 125.76) (end 158.72 128.17) (width 0.25) (layer "F.Cu") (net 45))
 (segment (start 158.795 121.697749) (end 159.837 122.739749) (width 0.25) (layer "F.Cu") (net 45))
 (segment (start 158.795 115.57) (end 158.795 121.697749) (width 0.25) (layer "F.Cu") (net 45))
 (segment (start 159.837 124.643) (end 158.72 125.76) (width 0.25) (layer "F.Cu") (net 45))
 (segment (start 159.837 122.739749) (end 159.837 124.643) (width 0.25) (layer "F.Cu") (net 45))
 (segment (start 157.48 122.556396) (end 157.48 124.46) (width 0.25) (layer "F.Cu") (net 44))
 (segment (start 156.18 125.76) (end 156.18 128.17) (width 0.25) (layer "F.Cu") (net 44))
 (segment (start 157.48 124.46) (end 156.18 125.76) (width 0.25) (layer "F.Cu") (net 44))
 (segment (start 156.255 121.331396) (end 157.48 122.556396) (width 0.25) (layer "F.Cu") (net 44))
 (segment (start 156.255 115.57) (end 156.255 121.331396) (width 0.25) (layer "F.Cu") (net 44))
 (segment (start 153.64 125.76) (end 153.64 128.17) (width 0.25) (layer "F.Cu") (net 43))
 (segment (start 153.715 115.57) (end 153.715 121.331396) (width 0.25) (layer "F.Cu") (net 43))
 (segment (start 154.94 122.556396) (end 154.94 124.46) (width 0.25) (layer "F.Cu") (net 43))
 (segment (start 153.715 121.331396) (end 154.94 122.556396) (width 0.25) (layer "F.Cu") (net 43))
 (segment (start 154.94 124.46) (end 153.64 125.76) (width 0.25) (layer "F.Cu") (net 43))
 (segment (start 152.4 122.556396) (end 152.4 124.46) (width 0.25) (layer "F.Cu") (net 42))
 (segment (start 151.1 125.76) (end 151.1 128.17) (width 0.25) (layer "F.Cu") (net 42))
 (segment (start 151.175 115.57) (end 151.175 121.331396) (width 0.25) (layer "F.Cu") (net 42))
 (segment (start 151.175 121.331396) (end 152.4 122.556396) (width 0.25) (layer "F.Cu") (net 42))
 (segment (start 152.4 124.46) (end 151.1 125.76) (width 0.25) (layer "F.Cu") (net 42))
 (segment (start 148.635 121.331396) (end 149.86 122.556396) (width 0.25) (layer "F.Cu") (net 41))
 (segment (start 149.86 124.46) (end 148.56 125.76) (width 0.25) (layer "F.Cu") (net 41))
 (segment (start 149.86 122.556396) (end 149.86 124.46) (width 0.25) (layer "F.Cu") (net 41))
 (segment (start 148.635 115.57) (end 148.635 121.331396) (width 0.25) (layer "F.Cu") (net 41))
 (segment (start 148.56 125.76) (end 148.56 128.17) (width 0.25) (layer "F.Cu") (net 41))
 (segment (start 146.095 115.57) (end 146.095 121.331396) (width 0.25) (layer "F.Cu") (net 40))
 (segment (start 146.02 125.76) (end 146.02 128.17) (width 0.25) (layer "F.Cu") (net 40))
 (segment (start 147.32 124.46) (end 146.02 125.76) (width 0.25) (layer "F.Cu") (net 40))
 (segment (start 147.32 122.556396) (end 147.32 124.46) (width 0.25) (layer "F.Cu") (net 40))
 (segment (start 146.095 121.331396) (end 147.32 122.556396) (width 0.25) (layer "F.Cu") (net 40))
 (segment (start 143.48 125.76) (end 143.48 128.17) (width 0.25) (layer "F.Cu") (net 39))
 (segment (start 143.555 121.331396) (end 144.78 122.556396) (width 0.25) (layer "F.Cu") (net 39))
 (segment (start 144.78 124.46) (end 143.48 125.76) (width 0.25) (layer "F.Cu") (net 39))
 (segment (start 143.555 115.57) (end 143.555 121.331396) (width 0.25) (layer "F.Cu") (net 39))
 (segment (start 144.78 122.556396) (end 144.78 124.46) (width 0.25) (layer "F.Cu") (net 39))
 (segment (start 140.94 125.76) (end 140.94 128.17) (width 0.25) (layer "F.Cu") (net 38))
 (segment (start 141.015 121.331396) (end 142.24 122.556396) (width 0.25) (layer "F.Cu") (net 38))
 (segment (start 141.015 115.57) (end 141.015 121.331396) (width 0.25) (layer "F.Cu") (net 38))
 (segment (start 142.24 124.46) (end 140.94 125.76) (width 0.25) (layer "F.Cu") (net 38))
 (segment (start 142.24 122.556396) (end 142.24 124.46) (width 0.25) (layer "F.Cu") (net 38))
 (segment (start 138.475 115.57) (end 138.475 121.331396) (width 0.25) (layer "F.Cu") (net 37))
 (segment (start 138.475 121.331396) (end 139.7 122.556396) (width 0.25) (layer "F.Cu") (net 37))
 (segment (start 139.7 122.556396) (end 139.7 124.46) (width 0.25) (layer "F.Cu") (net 37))
 (segment (start 139.7 124.46) (end 138.4 125.76) (width 0.25) (layer "F.Cu") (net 37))
 (segment (start 138.4 125.76) (end 138.4 128.17) (width 0.25) (layer "F.Cu") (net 37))
 (segment (start 135.935 115.57) (end 135.935 121.697749) (width 0.25) (layer "F.Cu") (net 36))
 (segment (start 136.977 122.739749) (end 136.977 124.643) (width 0.25) (layer "F.Cu") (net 36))
 (segment (start 136.977 124.643) (end 135.86 125.76) (width 0.25) (layer "F.Cu") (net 36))
 (segment (start 135.935 121.697749) (end 136.977 122.739749) (width 0.25) (layer "F.Cu") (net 36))
 (segment (start 135.86 125.76) (end 135.86 128.17) (width 0.25) (layer "F.Cu") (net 36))
 (segment (start 133.32 125.76) (end 133.32 128.17) (width 0.25) (layer "F.Cu") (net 35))
 (segment (start 134.62 124.46) (end 133.32 125.76) (width 0.25) (layer "F.Cu") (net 35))
 (segment (start 134.62 122.556396) (end 134.62 124.46) (width 0.25) (layer "F.Cu") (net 35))
 (segment (start 133.395 115.57) (end 133.395 121.331396) (width 0.25) (layer "F.Cu") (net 35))
 (segment (start 133.395 121.331396) (end 134.62 122.556396) (width 0.25) (layer "F.Cu") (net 35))
 (segment (start 131.897 122.739749) (end 131.897 124.643) (width 0.25) (layer "F.Cu") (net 34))
 (segment (start 130.855 121.697749) (end 131.897 122.739749) (width 0.25) (layer "F.Cu") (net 34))
 (segment (start 131.897 124.643) (end 130.78 125.76) (width 0.25) (layer "F.Cu") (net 34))
 (segment (start 130.855 115.57) (end 130.855 121.697749) (width 0.25) (layer "F.Cu") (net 34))
 (segment (start 130.78 125.76) (end 130.78 128.17) (width 0.25) (layer "F.Cu") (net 34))
 (segment (start 128.24 125.76) (end 128.24 128.17) (width 0.25) (layer "F.Cu") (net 33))
 (segment (start 128.315 115.57) (end 128.315 121.331396) (width 0.25) (layer "F.Cu") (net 33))
 (segment (start 129.54 122.556396) (end 129.54 124.46) (width 0.25) (layer "F.Cu") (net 33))
 (segment (start 129.54 124.46) (end 128.24 125.76) (width 0.25) (layer "F.Cu") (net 33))
 (segment (start 128.315 121.331396) (end 129.54 122.556396) (width 0.25) (layer "F.Cu") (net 33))
 (segment (start 125.775 121.697749) (end 126.817 122.739749) (width 0.25) (layer "F.Cu") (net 32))
 (segment (start 126.817 124.643) (end 125.7 125.76) (width 0.25) (layer "F.Cu") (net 32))
 (segment (start 126.817 122.739749) (end 126.817 124.643) (width 0.25) (layer "F.Cu") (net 32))
 (segment (start 125.775 115.57) (end 125.775 121.697749) (width 0.25) (layer "F.Cu") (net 32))
 (segment (start 125.7 125.76) (end 125.7 128.17) (width 0.25) (layer "F.Cu") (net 32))
 (segment (start 120.62 125.882302) (end 120.62 128.17) (width 0.25) (layer "F.Cu") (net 31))
 (segment (start 121.9258 122.672898) (end 121.9258 124.576502) (width 0.25) (layer "F.Cu") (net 31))
 (segment (start 120.7008 121.447898) (end 121.9258 122.672898) (width 0.25) (layer "F.Cu") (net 31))
 (segment (start 120.7008 115.686502) (end 120.7008 121.447898) (width 0.25) (layer "F.Cu") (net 31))
 (segment (start 121.9258 124.576502) (end 120.62 125.882302) (width 0.25) (layer "F.Cu") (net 31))
 (segment (start 118.155 121.331396) (end 119.38 122.556396) (width 0.25) (layer "F.Cu") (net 30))
 (segment (start 118.08 125.76) (end 118.08 128.17) (width 0.25) (layer "F.Cu") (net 30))
 (segment (start 118.155 115.57) (end 118.155 121.331396) (width 0.25) (layer "F.Cu") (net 30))
 (segment (start 119.38 124.46) (end 118.08 125.76) (width 0.25) (layer "F.Cu") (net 30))
 (segment (start 119.38 122.556396) (end 119.38 124.46) (width 0.25) (layer "F.Cu") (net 30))
 (segment (start 116.84 124.46) (end 115.54 125.76) (width 0.25) (layer "F.Cu") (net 29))
 (segment (start 115.615 115.57) (end 115.615 121.331396) (width 0.25) (layer "F.Cu") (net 29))
 (segment (start 115.54 125.76) (end 115.54 128.17) (width 0.25) (layer "F.Cu") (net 29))
 (segment (start 115.615 121.331396) (end 116.84 122.556396) (width 0.25) (layer "F.Cu") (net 29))
 (segment (start 116.84 122.556396) (end 116.84 124.46) (width 0.25) (layer "F.Cu") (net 29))
 (segment (start 113.075 115.57) (end 113.075 121.331396) (width 0.25) (layer "F.Cu") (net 28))
 (segment (start 113.075 121.331396) (end 114.3 122.556396) (width 0.25) (layer "F.Cu") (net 28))
 (segment (start 113 125.76) (end 113 128.17) (width 0.25) (layer "F.Cu") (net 28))
 (segment (start 114.3 124.46) (end 113 125.76) (width 0.25) (layer "F.Cu") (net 28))
 (segment (start 114.3 122.556396) (end 114.3 124.46) (width 0.25) (layer "F.Cu") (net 28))
 (segment (start 176.575 121.331396) (end 177.8 122.556396) (width 0.25) (layer "F.Cu") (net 52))
 (segment (start 176.575 115.57) (end 176.575 121.331396) (width 0.25) (layer "F.Cu") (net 52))
 (segment (start 177.8 122.556396) (end 177.8 124.46) (width 0.25) (layer "F.Cu") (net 52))
 (segment (start 176.5 125.76) (end 176.5 128.17) (width 0.25) (layer "F.Cu") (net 52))
 (segment (start 177.8 124.46) (end 176.5 125.76) (width 0.25) (layer "F.Cu") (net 52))
 (segment (start 181.655 115.57) (end 181.655 121.331396) (width 0.25) (layer "F.Cu") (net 54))
 (segment (start 181.58 125.76) (end 181.58 128.17) (width 0.25) (layer "F.Cu") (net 54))
 (segment (start 182.88 124.46) (end 181.58 125.76) (width 0.25) (layer "F.Cu") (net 54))
 (segment (start 182.88 122.556396) (end 182.88 124.46) (width 0.25) (layer "F.Cu") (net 54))
 (segment (start 181.655 121.331396) (end 182.88 122.556396) (width 0.25) (layer "F.Cu") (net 54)))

